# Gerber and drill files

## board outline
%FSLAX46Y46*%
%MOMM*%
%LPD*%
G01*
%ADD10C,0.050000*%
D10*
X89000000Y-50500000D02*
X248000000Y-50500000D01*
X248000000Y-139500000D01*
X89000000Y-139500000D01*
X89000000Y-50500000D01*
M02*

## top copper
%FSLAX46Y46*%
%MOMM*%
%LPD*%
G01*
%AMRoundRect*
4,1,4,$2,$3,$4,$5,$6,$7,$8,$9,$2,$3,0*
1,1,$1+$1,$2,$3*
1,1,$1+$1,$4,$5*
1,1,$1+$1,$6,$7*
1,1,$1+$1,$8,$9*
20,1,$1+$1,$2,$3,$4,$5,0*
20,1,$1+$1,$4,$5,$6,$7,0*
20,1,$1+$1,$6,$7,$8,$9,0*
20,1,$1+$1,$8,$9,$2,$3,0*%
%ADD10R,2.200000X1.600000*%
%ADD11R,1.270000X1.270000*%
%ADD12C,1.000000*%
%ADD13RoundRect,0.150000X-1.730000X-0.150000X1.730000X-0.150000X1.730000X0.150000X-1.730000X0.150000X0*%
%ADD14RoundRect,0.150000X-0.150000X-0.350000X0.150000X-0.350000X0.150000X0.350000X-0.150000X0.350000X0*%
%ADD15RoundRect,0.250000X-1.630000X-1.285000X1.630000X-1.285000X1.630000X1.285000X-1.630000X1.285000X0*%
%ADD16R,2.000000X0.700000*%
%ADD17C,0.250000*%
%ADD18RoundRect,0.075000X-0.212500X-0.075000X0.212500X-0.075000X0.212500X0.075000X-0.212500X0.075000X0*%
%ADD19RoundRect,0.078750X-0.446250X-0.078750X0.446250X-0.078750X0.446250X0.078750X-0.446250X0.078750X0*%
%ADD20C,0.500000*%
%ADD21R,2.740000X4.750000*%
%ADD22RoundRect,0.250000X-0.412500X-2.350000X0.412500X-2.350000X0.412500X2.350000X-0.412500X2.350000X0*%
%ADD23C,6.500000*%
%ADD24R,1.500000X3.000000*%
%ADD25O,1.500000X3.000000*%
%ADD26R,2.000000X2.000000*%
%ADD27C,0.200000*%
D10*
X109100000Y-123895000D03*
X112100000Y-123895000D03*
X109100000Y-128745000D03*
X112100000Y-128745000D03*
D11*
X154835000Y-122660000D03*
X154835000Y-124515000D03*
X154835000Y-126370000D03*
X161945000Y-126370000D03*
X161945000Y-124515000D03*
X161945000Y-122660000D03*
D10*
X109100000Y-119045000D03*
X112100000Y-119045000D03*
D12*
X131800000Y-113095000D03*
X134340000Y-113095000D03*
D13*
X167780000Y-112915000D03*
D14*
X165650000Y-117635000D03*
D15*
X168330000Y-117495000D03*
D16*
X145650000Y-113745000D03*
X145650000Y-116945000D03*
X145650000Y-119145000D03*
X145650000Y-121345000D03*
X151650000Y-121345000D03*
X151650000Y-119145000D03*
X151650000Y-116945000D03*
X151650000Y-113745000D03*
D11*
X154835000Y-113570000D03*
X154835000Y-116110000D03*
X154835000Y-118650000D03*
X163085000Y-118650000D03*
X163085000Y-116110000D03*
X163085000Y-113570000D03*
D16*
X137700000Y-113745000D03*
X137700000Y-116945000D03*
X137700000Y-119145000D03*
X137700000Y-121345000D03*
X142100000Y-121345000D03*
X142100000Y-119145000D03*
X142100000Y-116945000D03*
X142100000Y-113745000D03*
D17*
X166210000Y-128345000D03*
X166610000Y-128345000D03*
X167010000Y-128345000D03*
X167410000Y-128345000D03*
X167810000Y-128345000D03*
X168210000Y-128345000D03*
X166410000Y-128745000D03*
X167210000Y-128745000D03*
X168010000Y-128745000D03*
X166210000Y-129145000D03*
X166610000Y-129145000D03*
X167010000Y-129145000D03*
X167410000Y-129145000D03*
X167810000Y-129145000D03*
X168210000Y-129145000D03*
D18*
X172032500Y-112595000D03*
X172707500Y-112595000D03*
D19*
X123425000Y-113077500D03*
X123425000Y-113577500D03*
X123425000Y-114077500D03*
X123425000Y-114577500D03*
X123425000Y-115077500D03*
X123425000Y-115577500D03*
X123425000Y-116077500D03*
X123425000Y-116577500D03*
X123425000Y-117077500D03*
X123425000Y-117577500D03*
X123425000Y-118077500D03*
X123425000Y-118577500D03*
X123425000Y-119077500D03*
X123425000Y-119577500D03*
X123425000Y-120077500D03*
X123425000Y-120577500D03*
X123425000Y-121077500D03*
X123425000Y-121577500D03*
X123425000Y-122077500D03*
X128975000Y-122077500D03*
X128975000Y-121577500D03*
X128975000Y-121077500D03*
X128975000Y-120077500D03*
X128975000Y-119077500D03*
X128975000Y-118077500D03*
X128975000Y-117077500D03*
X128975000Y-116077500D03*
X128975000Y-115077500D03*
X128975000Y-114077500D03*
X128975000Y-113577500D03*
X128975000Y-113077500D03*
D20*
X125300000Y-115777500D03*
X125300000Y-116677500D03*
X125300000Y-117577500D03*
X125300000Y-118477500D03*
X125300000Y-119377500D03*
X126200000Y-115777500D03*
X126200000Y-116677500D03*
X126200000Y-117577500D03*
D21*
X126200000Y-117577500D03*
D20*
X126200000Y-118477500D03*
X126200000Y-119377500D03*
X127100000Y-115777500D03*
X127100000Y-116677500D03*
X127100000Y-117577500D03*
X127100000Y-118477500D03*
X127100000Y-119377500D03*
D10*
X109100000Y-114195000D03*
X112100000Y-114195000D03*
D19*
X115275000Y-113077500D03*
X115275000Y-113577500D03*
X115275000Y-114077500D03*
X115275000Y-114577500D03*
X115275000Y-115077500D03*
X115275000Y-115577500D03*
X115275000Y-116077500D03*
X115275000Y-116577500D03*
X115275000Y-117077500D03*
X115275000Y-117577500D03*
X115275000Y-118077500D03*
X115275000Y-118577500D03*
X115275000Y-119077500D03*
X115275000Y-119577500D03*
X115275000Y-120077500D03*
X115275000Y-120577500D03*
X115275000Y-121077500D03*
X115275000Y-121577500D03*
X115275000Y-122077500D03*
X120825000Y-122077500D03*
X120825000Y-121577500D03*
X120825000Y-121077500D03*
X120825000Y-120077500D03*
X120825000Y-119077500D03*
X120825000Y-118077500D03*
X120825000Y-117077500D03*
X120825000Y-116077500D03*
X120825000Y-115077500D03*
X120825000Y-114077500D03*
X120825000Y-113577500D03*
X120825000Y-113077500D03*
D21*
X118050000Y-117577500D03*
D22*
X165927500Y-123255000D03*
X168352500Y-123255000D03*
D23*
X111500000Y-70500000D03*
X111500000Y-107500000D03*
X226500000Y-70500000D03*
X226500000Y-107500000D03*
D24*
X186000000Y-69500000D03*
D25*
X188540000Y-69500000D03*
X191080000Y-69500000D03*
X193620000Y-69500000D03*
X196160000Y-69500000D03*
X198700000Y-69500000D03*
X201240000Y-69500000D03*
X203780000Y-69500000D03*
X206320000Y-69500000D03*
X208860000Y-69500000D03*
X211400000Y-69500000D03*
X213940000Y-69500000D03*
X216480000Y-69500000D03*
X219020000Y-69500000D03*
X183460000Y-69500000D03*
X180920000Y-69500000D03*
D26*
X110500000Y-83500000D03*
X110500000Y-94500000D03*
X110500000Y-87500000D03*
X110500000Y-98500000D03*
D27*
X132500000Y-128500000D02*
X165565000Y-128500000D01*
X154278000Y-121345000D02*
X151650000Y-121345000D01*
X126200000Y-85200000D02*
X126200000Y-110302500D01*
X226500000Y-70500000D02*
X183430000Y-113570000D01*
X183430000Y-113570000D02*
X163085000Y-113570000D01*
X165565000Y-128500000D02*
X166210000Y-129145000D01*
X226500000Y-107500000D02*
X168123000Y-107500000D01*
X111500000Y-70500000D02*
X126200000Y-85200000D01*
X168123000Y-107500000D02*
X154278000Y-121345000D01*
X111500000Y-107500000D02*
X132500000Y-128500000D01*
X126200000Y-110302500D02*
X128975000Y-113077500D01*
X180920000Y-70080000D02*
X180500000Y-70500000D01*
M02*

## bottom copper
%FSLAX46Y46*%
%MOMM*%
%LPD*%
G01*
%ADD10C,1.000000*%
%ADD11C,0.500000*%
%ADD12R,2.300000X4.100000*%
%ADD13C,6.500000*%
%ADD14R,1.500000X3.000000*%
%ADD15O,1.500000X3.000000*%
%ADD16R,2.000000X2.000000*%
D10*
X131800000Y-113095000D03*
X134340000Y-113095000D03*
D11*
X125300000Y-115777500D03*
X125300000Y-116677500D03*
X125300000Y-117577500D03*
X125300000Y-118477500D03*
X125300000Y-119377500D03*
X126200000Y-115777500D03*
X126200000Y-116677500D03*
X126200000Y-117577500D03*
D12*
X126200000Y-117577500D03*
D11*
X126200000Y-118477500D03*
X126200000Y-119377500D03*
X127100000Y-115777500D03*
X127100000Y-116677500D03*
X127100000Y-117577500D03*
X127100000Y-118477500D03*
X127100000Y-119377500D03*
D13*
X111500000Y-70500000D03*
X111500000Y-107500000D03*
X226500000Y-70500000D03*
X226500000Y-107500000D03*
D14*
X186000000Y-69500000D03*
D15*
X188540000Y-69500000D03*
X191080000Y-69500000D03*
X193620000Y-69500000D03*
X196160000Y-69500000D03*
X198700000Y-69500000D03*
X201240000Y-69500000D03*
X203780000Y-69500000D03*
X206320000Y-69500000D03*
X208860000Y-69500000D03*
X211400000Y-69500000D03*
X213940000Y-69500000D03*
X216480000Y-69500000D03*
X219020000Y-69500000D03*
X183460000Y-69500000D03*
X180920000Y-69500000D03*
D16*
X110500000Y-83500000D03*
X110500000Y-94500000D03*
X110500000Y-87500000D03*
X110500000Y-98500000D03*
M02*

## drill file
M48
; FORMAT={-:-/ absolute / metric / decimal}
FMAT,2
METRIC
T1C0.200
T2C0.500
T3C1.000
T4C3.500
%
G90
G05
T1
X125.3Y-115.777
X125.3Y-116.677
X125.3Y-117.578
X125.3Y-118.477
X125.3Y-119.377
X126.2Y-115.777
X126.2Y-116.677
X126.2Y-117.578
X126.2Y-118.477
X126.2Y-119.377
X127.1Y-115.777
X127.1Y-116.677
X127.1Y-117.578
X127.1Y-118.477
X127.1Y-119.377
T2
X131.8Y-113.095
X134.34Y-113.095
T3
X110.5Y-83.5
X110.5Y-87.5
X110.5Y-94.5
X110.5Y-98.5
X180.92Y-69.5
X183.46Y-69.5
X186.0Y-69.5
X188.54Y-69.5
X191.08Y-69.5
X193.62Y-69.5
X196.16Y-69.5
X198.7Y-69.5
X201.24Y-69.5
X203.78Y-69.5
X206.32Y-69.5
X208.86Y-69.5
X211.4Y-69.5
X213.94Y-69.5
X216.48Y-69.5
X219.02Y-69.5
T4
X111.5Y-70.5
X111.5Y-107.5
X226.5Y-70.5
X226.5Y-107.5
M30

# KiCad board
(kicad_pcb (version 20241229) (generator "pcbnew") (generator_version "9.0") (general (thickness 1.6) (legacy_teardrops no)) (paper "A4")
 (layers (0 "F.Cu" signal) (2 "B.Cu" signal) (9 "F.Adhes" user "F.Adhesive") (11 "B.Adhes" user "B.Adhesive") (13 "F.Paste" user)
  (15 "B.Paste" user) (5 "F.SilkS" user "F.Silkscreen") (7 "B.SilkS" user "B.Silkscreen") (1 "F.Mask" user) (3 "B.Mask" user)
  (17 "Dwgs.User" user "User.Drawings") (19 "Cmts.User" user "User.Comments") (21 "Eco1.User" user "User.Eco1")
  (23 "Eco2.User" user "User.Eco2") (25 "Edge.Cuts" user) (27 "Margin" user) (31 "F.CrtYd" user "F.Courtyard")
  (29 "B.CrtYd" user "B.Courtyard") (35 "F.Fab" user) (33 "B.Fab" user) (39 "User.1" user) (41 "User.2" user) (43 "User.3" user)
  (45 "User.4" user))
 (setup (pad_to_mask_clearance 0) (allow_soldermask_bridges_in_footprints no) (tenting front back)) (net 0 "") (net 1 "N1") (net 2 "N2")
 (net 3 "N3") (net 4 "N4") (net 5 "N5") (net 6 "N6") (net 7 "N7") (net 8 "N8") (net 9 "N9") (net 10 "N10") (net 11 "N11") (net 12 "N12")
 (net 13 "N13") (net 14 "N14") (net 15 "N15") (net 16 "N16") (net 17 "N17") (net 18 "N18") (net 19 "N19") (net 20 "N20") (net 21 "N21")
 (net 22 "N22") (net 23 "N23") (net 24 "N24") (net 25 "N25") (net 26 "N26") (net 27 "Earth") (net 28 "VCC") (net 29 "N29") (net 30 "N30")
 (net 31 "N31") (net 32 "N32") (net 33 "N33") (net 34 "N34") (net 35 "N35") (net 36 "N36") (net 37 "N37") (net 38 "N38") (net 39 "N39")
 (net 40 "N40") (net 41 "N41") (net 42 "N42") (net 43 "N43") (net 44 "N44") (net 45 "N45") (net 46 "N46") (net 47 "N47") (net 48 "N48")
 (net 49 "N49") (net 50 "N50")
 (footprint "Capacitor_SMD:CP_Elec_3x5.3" (layer "F.Cu") (at 110.6 123.895)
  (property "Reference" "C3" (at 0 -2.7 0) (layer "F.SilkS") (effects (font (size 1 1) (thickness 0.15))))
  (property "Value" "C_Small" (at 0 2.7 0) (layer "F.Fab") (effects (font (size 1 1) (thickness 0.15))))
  (pad "1" smd rect (at -1.5 0) (size 2.2 1.6) (layers "F.Cu" "F.Mask" "F.Paste") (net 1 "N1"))
  (pad "2" smd rect (at 1.5 0) (size 2.2 1.6) (layers "F.Cu" "F.Mask" "F.Paste") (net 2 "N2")))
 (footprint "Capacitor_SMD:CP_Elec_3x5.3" (layer "F.Cu") (at 110.6 128.745)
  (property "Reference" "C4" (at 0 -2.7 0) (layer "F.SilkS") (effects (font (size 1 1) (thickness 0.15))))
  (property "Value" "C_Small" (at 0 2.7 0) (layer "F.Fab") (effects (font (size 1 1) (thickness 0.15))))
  (pad "1" smd rect (at -1.5 0) (size 2.2 1.6) (layers "F.Cu" "F.Mask" "F.Paste") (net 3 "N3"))
  (pad "2" smd rect (at 1.5 0) (size 2.2 1.6) (layers "F.Cu" "F.Mask" "F.Paste") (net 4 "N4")))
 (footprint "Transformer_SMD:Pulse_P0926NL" (layer "F.Cu") (at 158.39 124.515)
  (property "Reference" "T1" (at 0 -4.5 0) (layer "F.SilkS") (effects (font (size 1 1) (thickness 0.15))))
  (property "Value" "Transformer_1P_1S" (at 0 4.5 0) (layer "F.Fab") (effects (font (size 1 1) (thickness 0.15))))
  (pad "1" smd rect (at -3.555 -1.855) (size 1.27 1.27) (layers "F.Cu" "F.Mask" "F.Paste") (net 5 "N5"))
  (pad "2" smd rect (at -3.555 0) (size 1.27 1.27) (layers "F.Cu" "F.Mask" "F.Paste") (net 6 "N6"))
  (pad "3" smd rect (at -3.555 1.855) (size 1.27 1.27) (layers "F.Cu" "F.Mask" "F.Paste") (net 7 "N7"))
  (pad "4" smd rect (at 3.555 1.855) (size 1.27 1.27) (layers "F.Cu" "F.Mask" "F.Paste") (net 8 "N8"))
  (pad "5" smd rect (at 3.555 0) (size 1.27 1.27) (layers "F.Cu" "F.Mask" "F.Paste"))
  (pad "6" smd rect (at 3.555 -1.855) (size 1.27 1.27) (layers "F.Cu" "F.Mask" "F.Paste")))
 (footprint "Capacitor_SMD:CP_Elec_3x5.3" (layer "F.Cu") (at 110.6 119.045)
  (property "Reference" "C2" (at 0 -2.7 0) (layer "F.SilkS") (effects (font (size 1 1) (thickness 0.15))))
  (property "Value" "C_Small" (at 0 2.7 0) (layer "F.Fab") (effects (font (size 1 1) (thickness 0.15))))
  (pad "1" smd rect (at -1.5 0) (size 2.2 1.6) (layers "F.Cu" "F.Mask" "F.Paste") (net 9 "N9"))
  (pad "2" smd rect (at 1.5 0) (size 2.2 1.6) (layers "F.Cu" "F.Mask" "F.Paste") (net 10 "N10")))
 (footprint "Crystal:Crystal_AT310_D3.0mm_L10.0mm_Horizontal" (layer "F.Cu") (at 131.8 113.095)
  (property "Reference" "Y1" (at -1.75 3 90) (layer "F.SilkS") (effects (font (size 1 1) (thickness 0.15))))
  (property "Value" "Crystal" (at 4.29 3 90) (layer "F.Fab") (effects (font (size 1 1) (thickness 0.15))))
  (pad "1" thru_hole circle (at 0 0) (size 1 1) (drill 0.5) (layers "*.Cu" "*.Mask") (remove_unused_layers no) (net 10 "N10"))
  (pad "2" thru_hole circle (at 2.54 0) (size 1 1) (drill 0.5) (layers "*.Cu" "*.Mask") (remove_unused_layers no) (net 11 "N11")))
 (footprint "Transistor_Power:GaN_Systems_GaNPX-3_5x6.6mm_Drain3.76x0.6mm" (layer "F.Cu") (at 167.78 115.825)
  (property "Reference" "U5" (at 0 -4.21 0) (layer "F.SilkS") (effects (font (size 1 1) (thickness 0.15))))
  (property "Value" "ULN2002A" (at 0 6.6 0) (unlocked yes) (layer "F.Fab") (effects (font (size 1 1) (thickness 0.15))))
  (pad "" smd roundrect (at -0.34 0.9525) (size 1.58 1.235) (layers "F.Paste") (roundrect_rratio 0.2024291498))
  (pad "" smd roundrect (at -0.34 2.3875) (size 1.58 1.235) (layers "F.Paste") (roundrect_rratio 0.2024291498))
  (pad "" smd roundrect (at 1.44 0.9525) (size 1.58 1.235) (layers "F.Paste") (roundrect_rratio 0.2024291498))
  (pad "" smd roundrect (at 1.44 2.3875) (size 1.58 1.235) (layers "F.Paste") (roundrect_rratio 0.2024291498))
  (pad "1" smd roundrect (at 0 -2.91) (size 3.76 0.6) (layers "F.Cu" "F.Mask" "F.Paste") (roundrect_rratio 0.25) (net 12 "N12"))
  (pad "2" smd roundrect (at -2.13 1.81) (size 0.6 1) (layers "F.Cu" "F.Mask" "F.Paste") (roundrect_rratio 0.25) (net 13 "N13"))
  (pad "3" smd roundrect (at 0.55 1.67) (size 3.76 3.07) (layers "F.Cu" "F.Mask") (roundrect_rratio 0.08143322476) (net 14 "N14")))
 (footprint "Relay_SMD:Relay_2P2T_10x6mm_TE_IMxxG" (layer "F.Cu") (at 148.65 117.545)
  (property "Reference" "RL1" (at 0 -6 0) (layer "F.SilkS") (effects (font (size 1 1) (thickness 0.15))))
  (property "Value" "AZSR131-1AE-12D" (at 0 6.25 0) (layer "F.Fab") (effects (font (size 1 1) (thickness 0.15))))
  (pad "1" smd rect (at -3 -3.8) (size 2 0.7) (layers "F.Cu" "F.Mask" "F.Paste") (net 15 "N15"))
  (pad "2" smd rect (at -3 -0.6) (size 2 0.7) (layers "F.Cu" "F.Mask" "F.Paste") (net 2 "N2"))
  (pad "3" smd rect (at -3 1.6) (size 2 0.7) (layers "F.Cu" "F.Mask" "F.Paste") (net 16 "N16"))
  (pad "4" smd rect (at -3 3.8) (size 2 0.7) (layers "F.Cu" "F.Mask" "F.Paste") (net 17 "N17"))
  (pad "5" smd rect (at 3 3.8) (size 2 0.7) (layers "F.Cu" "F.Mask" "F.Paste"))
  (pad "6" smd rect (at 3 1.6) (size 2 0.7) (layers "F.Cu" "F.Mask" "F.Paste"))
  (pad "7" smd rect (at 3 -0.6) (size 2 0.7) (layers "F.Cu" "F.Mask" "F.Paste"))
  (pad "8" smd rect (at 3 -3.8) (size 2 0.7) (layers "F.Cu" "F.Mask" "F.Paste")))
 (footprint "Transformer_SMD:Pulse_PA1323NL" (layer "F.Cu") (at 158.96 116.11)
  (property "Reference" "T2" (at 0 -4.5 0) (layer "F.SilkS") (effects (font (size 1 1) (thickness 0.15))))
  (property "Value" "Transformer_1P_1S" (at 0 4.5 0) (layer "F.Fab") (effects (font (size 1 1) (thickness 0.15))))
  (pad "1" smd rect (at -4.125 -2.54) (size 1.27 1.27) (layers "F.Cu" "F.Mask" "F.Paste") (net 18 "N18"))
  (pad "2" smd rect (at -4.125 0) (size 1.27 1.27) (layers "F.Cu" "F.Mask" "F.Paste") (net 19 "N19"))
  (pad "3" smd rect (at -4.125 2.54) (size 1.27 1.27) (layers "F.Cu" "F.Mask" "F.Paste") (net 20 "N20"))
  (pad "4" smd rect (at 4.125 2.54) (size 1.27 1.27) (layers "F.Cu" "F.Mask" "F.Paste") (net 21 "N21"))
  (pad "5" smd rect (at 4.125 0) (size 1.27 1.27) (layers "F.Cu" "F.Mask" "F.Paste"))
  (pad "6" smd rect (at 4.125 -2.54) (size 1.27 1.27) (layers "F.Cu" "F.Mask" "F.Paste")))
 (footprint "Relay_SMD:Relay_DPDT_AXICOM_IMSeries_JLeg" (layer "F.Cu") (at 139.9 117.545)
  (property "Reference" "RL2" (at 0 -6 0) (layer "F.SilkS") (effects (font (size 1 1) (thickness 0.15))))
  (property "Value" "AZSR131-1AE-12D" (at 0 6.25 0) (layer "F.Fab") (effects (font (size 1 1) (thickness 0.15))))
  (pad "1" smd rect (at -2.2 -3.8) (size 2 0.7) (layers "F.Cu" "F.Mask" "F.Paste") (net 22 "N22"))
  (pad "2" smd rect (at -2.2 -0.6) (size 2 0.7) (layers "F.Cu" "F.Mask" "F.Paste") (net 16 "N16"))
  (pad "3" smd rect (at -2.2 1.6) (size 2 0.7) (layers "F.Cu" "F.Mask" "F.Paste") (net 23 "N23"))
  (pad "4" smd rect (at -2.2 3.8) (size 2 0.7) (layers "F.Cu" "F.Mask" "F.Paste") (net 4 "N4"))
  (pad "5" smd rect (at 2.2 3.8) (size 2 0.7) (layers "F.Cu" "F.Mask" "F.Paste"))
  (pad "6" smd rect (at 2.2 1.6) (size 2 0.7) (layers "F.Cu" "F.Mask" "F.Paste"))
  (pad "7" smd rect (at 2.2 -0.6) (size 2 0.7) (layers "F.Cu" "F.Mask" "F.Paste"))
  (pad "8" smd rect (at 2.2 -3.8) (size 2 0.7) (layers "F.Cu" "F.Mask" "F.Paste")))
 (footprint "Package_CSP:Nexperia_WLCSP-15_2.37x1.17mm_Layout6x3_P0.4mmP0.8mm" (layer "F.Cu") (at 167.21 128.745)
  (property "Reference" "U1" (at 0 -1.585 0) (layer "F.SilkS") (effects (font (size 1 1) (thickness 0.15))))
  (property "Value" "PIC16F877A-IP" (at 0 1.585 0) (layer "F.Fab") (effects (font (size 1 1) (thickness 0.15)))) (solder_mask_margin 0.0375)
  (pad "A1" smd circle (at -1 -0.4) (size 0.25 0.25) (layers "F.Cu" "F.Mask" "F.Paste"))
  (pad "A2" smd circle (at -0.6 -0.4) (size 0.25 0.25) (layers "F.Cu" "F.Mask" "F.Paste"))
  (pad "A3" smd circle (at -0.2 -0.4) (size 0.25 0.25) (layers "F.Cu" "F.Mask" "F.Paste"))
  (pad "A4" smd circle (at 0.2 -0.4) (size 0.25 0.25) (layers "F.Cu" "F.Mask" "F.Paste"))
  (pad "A5" smd circle (at 0.6 -0.4) (size 0.25 0.25) (layers "F.Cu" "F.Mask" "F.Paste"))
  (pad "A6" smd circle (at 1 -0.4) (size 0.25 0.25) (layers "F.Cu" "F.Mask" "F.Paste"))
  (pad "B1" smd circle (at -0.8 0) (size 0.25 0.25) (layers "F.Cu" "F.Mask" "F.Paste"))
  (pad "B2" smd circle (at 0 0) (size 0.25 0.25) (layers "F.Cu" "F.Mask" "F.Paste"))
  (pad "B3" smd circle (at 0.8 0) (size 0.25 0.25) (layers "F.Cu" "F.Mask" "F.Paste"))
  (pad "C1" smd circle (at -1 0.4) (size 0.25 0.25) (layers "F.Cu" "F.Mask" "F.Paste"))
  (pad "C2" smd circle (at -0.6 0.4) (size 0.25 0.25) (layers "F.Cu" "F.Mask" "F.Paste"))
  (pad "C3" smd circle (at -0.2 0.4) (size 0.25 0.25) (layers "F.Cu" "F.Mask" "F.Paste"))
  (pad "C4" smd circle (at 0.2 0.4) (size 0.25 0.25) (layers "F.Cu" "F.Mask" "F.Paste"))
  (pad "C5" smd circle (at 0.6 0.4) (size 0.25 0.25) (layers "F.Cu" "F.Mask" "F.Paste"))
  (pad "C6" smd circle (at 1 0.4) (size 0.25 0.25) (layers "F.Cu" "F.Mask" "F.Paste")))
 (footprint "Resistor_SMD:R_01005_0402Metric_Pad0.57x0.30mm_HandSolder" (layer "F.Cu") (at 172.37 112.595)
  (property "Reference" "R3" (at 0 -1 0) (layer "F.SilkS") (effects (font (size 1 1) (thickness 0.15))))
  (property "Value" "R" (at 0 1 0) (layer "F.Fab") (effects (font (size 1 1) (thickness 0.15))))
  (pad "" smd roundrect (at -0.3625 0) (size 0.41 0.27) (layers "F.Paste") (roundrect_rratio 0.25))
  (pad "" smd roundrect (at 0.3625 0) (size 0.41 0.27) (layers "F.Paste") (roundrect_rratio 0.25))
  (pad "1" smd roundrect (at -0.3375 0) (size 0.575 0.3) (layers "F.Cu" "F.Mask") (roundrect_rratio 0.25) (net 19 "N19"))
  (pad "2" smd roundrect (at 0.3375 0) (size 0.575 0.3) (layers "F.Cu" "F.Mask") (roundrect_rratio 0.25) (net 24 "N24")))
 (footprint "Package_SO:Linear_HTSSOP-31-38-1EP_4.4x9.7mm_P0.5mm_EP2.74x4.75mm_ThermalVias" (layer "F.Cu") (at 126.2 117.5775)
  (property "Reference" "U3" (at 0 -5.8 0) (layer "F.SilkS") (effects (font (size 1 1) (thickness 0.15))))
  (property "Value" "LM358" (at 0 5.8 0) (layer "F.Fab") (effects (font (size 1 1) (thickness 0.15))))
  (pad "" smd roundrect (at -0.685 -1.58) (size 1.1 1.28) (layers "F.Paste") (roundrect_rratio 0.227273))
  (pad "" smd roundrect (at -0.685 0) (size 1.1 1.28) (layers "F.Paste") (roundrect_rratio 0.227273))
  (pad "" smd roundrect (at -0.685 1.58) (size 1.1 1.28) (layers "F.Paste") (roundrect_rratio 0.227273))
  (pad "" smd roundrect (at 0.685 -1.58) (size 1.1 1.28) (layers "F.Paste") (roundrect_rratio 0.227273))
  (pad "" smd roundrect (at 0.685 0) (size 1.1 1.28) (layers "F.Paste") (roundrect_rratio 0.227273))
  (pad "" smd roundrect (at 0.685 1.58) (size 1.1 1.28) (layers "F.Paste") (roundrect_rratio 0.227273))
  (pad "1" smd roundrect (at -2.775 -4.5) (size 1.05 0.315) (layers "F.Cu" "F.Mask" "F.Paste") (roundrect_rratio 0.25) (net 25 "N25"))
  (pad "2" smd roundrect (at -2.775 -4) (size 1.05 0.315) (layers "F.Cu" "F.Mask" "F.Paste") (roundrect_rratio 0.25) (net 5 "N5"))
  (pad "3" smd roundrect (at -2.775 -3.5) (size 1.05 0.315) (layers "F.Cu" "F.Mask" "F.Paste") (roundrect_rratio 0.25) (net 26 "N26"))
  (pad "4" smd roundrect (at -2.775 -3) (size 1.05 0.315) (layers "F.Cu" "F.Mask" "F.Paste") (roundrect_rratio 0.25) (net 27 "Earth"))
  (pad "5" smd roundrect (at -2.775 -2.5) (size 1.05 0.315) (layers "F.Cu" "F.Mask" "F.Paste") (roundrect_rratio 0.25))
  (pad "6" smd roundrect (at -2.775 -2) (size 1.05 0.315) (layers "F.Cu" "F.Mask" "F.Paste") (roundrect_rratio 0.25))
  (pad "7" smd roundrect (at -2.775 -1.5) (size 1.05 0.315) (layers "F.Cu" "F.Mask" "F.Paste") (roundrect_rratio 0.25))
  (pad "8" smd roundrect (at -2.775 -1) (size 1.05 0.315) (layers "F.Cu" "F.Mask" "F.Paste") (roundrect_rratio 0.25) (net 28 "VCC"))
  (pad "9" smd roundrect (at -2.775 -0.5) (size 1.05 0.315) (layers "F.Cu" "F.Mask" "F.Paste") (roundrect_rratio 0.25))
  (pad "10" smd roundrect (at -2.775 0) (size 1.05 0.315) (layers "F.Cu" "F.Mask" "F.Paste") (roundrect_rratio 0.25))
  (pad "11" smd roundrect (at -2.775 0.5) (size 1.05 0.315) (layers "F.Cu" "F.Mask" "F.Paste") (roundrect_rratio 0.25))
  (pad "12" smd roundrect (at -2.775 1) (size 1.05 0.315) (layers "F.Cu" "F.Mask" "F.Paste") (roundrect_rratio 0.25))
  (pad "13" smd roundrect (at -2.775 1.5) (size 1.05 0.315) (layers "F.Cu" "F.Mask" "F.Paste") (roundrect_rratio 0.25))
  (pad "14" smd roundrect (at -2.775 2) (size 1.05 0.315) (layers "F.Cu" "F.Mask" "F.Paste") (roundrect_rratio 0.25))
  (pad "15" smd roundrect (at -2.775 2.5) (size 1.05 0.315) (layers "F.Cu" "F.Mask" "F.Paste") (roundrect_rratio 0.25))
  (pad "16" smd roundrect (at -2.775 3) (size 1.05 0.315) (layers "F.Cu" "F.Mask" "F.Paste") (roundrect_rratio 0.25))
  (pad "17" smd roundrect (at -2.775 3.5) (size 1.05 0.315) (layers "F.Cu" "F.Mask" "F.Paste") (roundrect_rratio 0.25))
  (pad "18" smd roundrect (at -2.775 4) (size 1.05 0.315) (layers "F.Cu" "F.Mask" "F.Paste") (roundrect_rratio 0.25))
  (pad "19" smd roundrect (at -2.775 4.5) (size 1.05 0.315) (layers "F.Cu" "F.Mask" "F.Paste") (roundrect_rratio 0.25))
  (pad "20" smd roundrect (at 2.775 4.5) (size 1.05 0.315) (layers "F.Cu" "F.Mask" "F.Paste") (roundrect_rratio 0.25))
  (pad "21" smd roundrect (at 2.775 4) (size 1.05 0.315) (layers "F.Cu" "F.Mask" "F.Paste") (roundrect_rratio 0.25))
  (pad "22" smd roundrect (at 2.775 3.5) (size 1.05 0.315) (layers "F.Cu" "F.Mask" "F.Paste") (roundrect_rratio 0.25))
  (pad "24" smd roundrect (at 2.775 2.5) (size 1.05 0.315) (layers "F.Cu" "F.Mask" "F.Paste") (roundrect_rratio 0.25))
  (pad "26" smd roundrect (at 2.775 1.5) (size 1.05 0.315) (layers "F.Cu" "F.Mask" "F.Paste") (roundrect_rratio 0.25))
  (pad "28" smd roundrect (at 2.775 0.5) (size 1.05 0.315) (layers "F.Cu" "F.Mask" "F.Paste") (roundrect_rratio 0.25))
  (pad "30" smd roundrect (at 2.775 -0.5) (size 1.05 0.315) (layers "F.Cu" "F.Mask" "F.Paste") (roundrect_rratio 0.25))
  (pad "32" smd roundrect (at 2.775 -1.5) (size 1.05 0.315) (layers "F.Cu" "F.Mask" "F.Paste") (roundrect_rratio 0.25))
  (pad "34" smd roundrect (at 2.775 -2.5) (size 1.05 0.315) (layers "F.Cu" "F.Mask" "F.Paste") (roundrect_rratio 0.25))
  (pad "36" smd roundrect (at 2.775 -3.5) (size 1.05 0.315) (layers "F.Cu" "F.Mask" "F.Paste") (roundrect_rratio 0.25))
  (pad "37" smd roundrect (at 2.775 -4) (size 1.05 0.315) (layers "F.Cu" "F.Mask" "F.Paste") (roundrect_rratio 0.25))
  (pad "38" smd roundrect (at 2.775 -4.5) (size 1.05 0.315) (layers "F.Cu" "F.Mask" "F.Paste") (roundrect_rratio 0.25))
  (pad "39" thru_hole circle (at -0.9 -1.8) (size 0.5 0.5) (drill 0.2) (layers "*.Cu") (remove_unused_layers no))
  (pad "39" thru_hole circle (at -0.9 -0.9) (size 0.5 0.5) (drill 0.2) (layers "*.Cu") (remove_unused_layers no))
  (pad "39" thru_hole circle (at -0.9 0) (size 0.5 0.5) (drill 0.2) (layers "*.Cu") (remove_unused_layers no))
  (pad "39" thru_hole circle (at -0.9 0.9) (size 0.5 0.5) (drill 0.2) (layers "*.Cu") (remove_unused_layers no))
  (pad "39" thru_hole circle (at -0.9 1.8) (size 0.5 0.5) (drill 0.2) (layers "*.Cu") (remove_unused_layers no))
  (pad "39" thru_hole circle (at 0 -1.8) (size 0.5 0.5) (drill 0.2) (layers "*.Cu") (remove_unused_layers no))
  (pad "39" thru_hole circle (at 0 -0.9) (size 0.5 0.5) (drill 0.2) (layers "*.Cu") (remove_unused_layers no))
  (pad "39" thru_hole circle (at 0 0) (size 0.5 0.5) (drill 0.2) (layers "*.Cu") (remove_unused_layers no))
  (pad "39" smd rect (at 0 0) (size 2.3 4.1) (layers "B.Cu") (zone_connect 2))
  (pad "39" smd rect (at 0 0) (size 2.74 4.75) (layers "F.Cu" "F.Mask") (zone_connect 2))
  (pad "39" thru_hole circle (at 0 0.9) (size 0.5 0.5) (drill 0.2) (layers "*.Cu") (remove_unused_layers no))
  (pad "39" thru_hole circle (at 0 1.8) (size 0.5 0.5) (drill 0.2) (layers "*.Cu") (remove_unused_layers no))
  (pad "39" thru_hole circle (at 0.9 -1.8) (size 0.5 0.5) (drill 0.2) (layers "*.Cu") (remove_unused_layers no))
  (pad "39" thru_hole circle (at 0.9 -0.9) (size 0.5 0.5) (drill 0.2) (layers "*.Cu") (remove_unused_layers no))
  (pad "39" thru_hole circle (at 0.9 0) (size 0.5 0.5) (drill 0.2) (layers "*.Cu") (remove_unused_layers no))
  (pad "39" thru_hole circle (at 0.9 0.9) (size 0.5 0.5) (drill 0.2) (layers "*.Cu") (remove_unused_layers no))
  (pad "39" thru_hole circle (at 0.9 1.8) (size 0.5 0.5) (drill 0.2) (layers "*.Cu") (remove_unused_layers no)))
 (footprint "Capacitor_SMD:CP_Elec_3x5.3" (layer "F.Cu") (at 110.6 114.195)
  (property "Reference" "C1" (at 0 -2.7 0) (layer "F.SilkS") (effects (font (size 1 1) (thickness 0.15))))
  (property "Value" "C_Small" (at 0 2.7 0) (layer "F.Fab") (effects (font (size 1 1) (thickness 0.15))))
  (pad "1" smd rect (at -1.5 0) (size 2.2 1.6) (layers "F.Cu" "F.Mask" "F.Paste") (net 11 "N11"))
  (pad "2" smd rect (at 1.5 0) (size 2.2 1.6) (layers "F.Cu" "F.Mask" "F.Paste") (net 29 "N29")))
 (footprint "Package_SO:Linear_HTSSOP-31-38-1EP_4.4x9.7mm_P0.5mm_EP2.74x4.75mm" (layer "F.Cu") (at 118.05 117.5775)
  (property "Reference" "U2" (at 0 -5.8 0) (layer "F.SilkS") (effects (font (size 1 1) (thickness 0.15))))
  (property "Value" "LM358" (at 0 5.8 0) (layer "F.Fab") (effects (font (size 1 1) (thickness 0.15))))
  (pad "" smd roundrect (at -0.685 -1.58) (size 1.1 1.28) (layers "F.Paste") (roundrect_rratio 0.227273))
  (pad "" smd roundrect (at -0.685 0) (size 1.1 1.28) (layers "F.Paste") (roundrect_rratio 0.227273))
  (pad "" smd roundrect (at -0.685 1.58) (size 1.1 1.28) (layers "F.Paste") (roundrect_rratio 0.227273))
  (pad "" smd roundrect (at 0.685 -1.58) (size 1.1 1.28) (layers "F.Paste") (roundrect_rratio 0.227273))
  (pad "" smd roundrect (at 0.685 0) (size 1.1 1.28) (layers "F.Paste") (roundrect_rratio 0.227273))
  (pad "" smd roundrect (at 0.685 1.58) (size 1.1 1.28) (layers "F.Paste") (roundrect_rratio 0.227273))
  (pad "1" smd roundrect (at -2.775 -4.5) (size 1.05 0.315) (layers "F.Cu" "F.Mask" "F.Paste") (roundrect_rratio 0.25))
  (pad "2" smd roundrect (at -2.775 -4) (size 1.05 0.315) (layers "F.Cu" "F.Mask" "F.Paste") (roundrect_rratio 0.25))
  (pad "3" smd roundrect (at -2.775 -3.5) (size 1.05 0.315) (layers "F.Cu" "F.Mask" "F.Paste") (roundrect_rratio 0.25))
  (pad "4" smd roundrect (at -2.775 -3) (size 1.05 0.315) (layers "F.Cu" "F.Mask" "F.Paste") (roundrect_rratio 0.25) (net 27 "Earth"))
  (pad "5" smd roundrect (at -2.775 -2.5) (size 1.05 0.315) (layers "F.Cu" "F.Mask" "F.Paste") (roundrect_rratio 0.25) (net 24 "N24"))
  (pad "6" smd roundrect (at -2.775 -2) (size 1.05 0.315) (layers "F.Cu" "F.Mask" "F.Paste") (roundrect_rratio 0.25) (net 18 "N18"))
  (pad "7" smd roundrect (at -2.775 -1.5) (size 1.05 0.315) (layers "F.Cu" "F.Mask" "F.Paste") (roundrect_rratio 0.25) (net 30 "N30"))
  (pad "8" smd roundrect (at -2.775 -1) (size 1.05 0.315) (layers "F.Cu" "F.Mask" "F.Paste") (roundrect_rratio 0.25) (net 28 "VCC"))
  (pad "9" smd roundrect (at -2.775 -0.5) (size 1.05 0.315) (layers "F.Cu" "F.Mask" "F.Paste") (roundrect_rratio 0.25))
  (pad "10" smd roundrect (at -2.775 0) (size 1.05 0.315) (layers "F.Cu" "F.Mask" "F.Paste") (roundrect_rratio 0.25))
  (pad "11" smd roundrect (at -2.775 0.5) (size 1.05 0.315) (layers "F.Cu" "F.Mask" "F.Paste") (roundrect_rratio 0.25))
  (pad "12" smd roundrect (at -2.775 1) (size 1.05 0.315) (layers "F.Cu" "F.Mask" "F.Paste") (roundrect_rratio 0.25))
  (pad "13" smd roundrect (at -2.775 1.5) (size 1.05 0.315) (layers "F.Cu" "F.Mask" "F.Paste") (roundrect_rratio 0.25))
  (pad "14" smd roundrect (at -2.775 2) (size 1.05 0.315) (layers "F.Cu" "F.Mask" "F.Paste") (roundrect_rratio 0.25))
  (pad "15" smd roundrect (at -2.775 2.5) (size 1.05 0.315) (layers "F.Cu" "F.Mask" "F.Paste") (roundrect_rratio 0.25))
  (pad "16" smd roundrect (at -2.775 3) (size 1.05 0.315) (layers "F.Cu" "F.Mask" "F.Paste") (roundrect_rratio 0.25))
  (pad "17" smd roundrect (at -2.775 3.5) (size 1.05 0.315) (layers "F.Cu" "F.Mask" "F.Paste") (roundrect_rratio 0.25))
  (pad "18" smd roundrect (at -2.775 4) (size 1.05 0.315) (layers "F.Cu" "F.Mask" "F.Paste") (roundrect_rratio 0.25))
  (pad "19" smd roundrect (at -2.775 4.5) (size 1.05 0.315) (layers "F.Cu" "F.Mask" "F.Paste") (roundrect_rratio 0.25))
  (pad "20" smd roundrect (at 2.775 4.5) (size 1.05 0.315) (layers "F.Cu" "F.Mask" "F.Paste") (roundrect_rratio 0.25))
  (pad "21" smd roundrect (at 2.775 4) (size 1.05 0.315) (layers "F.Cu" "F.Mask" "F.Paste") (roundrect_rratio 0.25))
  (pad "22" smd roundrect (at 2.775 3.5) (size 1.05 0.315) (layers "F.Cu" "F.Mask" "F.Paste") (roundrect_rratio 0.25))
  (pad "24" smd roundrect (at 2.775 2.5) (size 1.05 0.315) (layers "F.Cu" "F.Mask" "F.Paste") (roundrect_rratio 0.25))
  (pad "26" smd roundrect (at 2.775 1.5) (size 1.05 0.315) (layers "F.Cu" "F.Mask" "F.Paste") (roundrect_rratio 0.25))
  (pad "28" smd roundrect (at 2.775 0.5) (size 1.05 0.315) (layers "F.Cu" "F.Mask" "F.Paste") (roundrect_rratio 0.25))
  (pad "30" smd roundrect (at 2.775 -0.5) (size 1.05 0.315) (layers "F.Cu" "F.Mask" "F.Paste") (roundrect_rratio 0.25))
  (pad "32" smd roundrect (at 2.775 -1.5) (size 1.05 0.315) (layers "F.Cu" "F.Mask" "F.Paste") (roundrect_rratio 0.25))
  (pad "34" smd roundrect (at 2.775 -2.5) (size 1.05 0.315) (layers "F.Cu" "F.Mask" "F.Paste") (roundrect_rratio 0.25))
  (pad "36" smd roundrect (at 2.775 -3.5) (size 1.05 0.315) (layers "F.Cu" "F.Mask" "F.Paste") (roundrect_rratio 0.25))
  (pad "37" smd roundrect (at 2.775 -4) (size 1.05 0.315) (layers "F.Cu" "F.Mask" "F.Paste") (roundrect_rratio 0.25))
  (pad "38" smd roundrect (at 2.775 -4.5) (size 1.05 0.315) (layers "F.Cu" "F.Mask" "F.Paste") (roundrect_rratio 0.25))
  (pad "39" smd rect (at 0 0) (size 2.74 4.75) (layers "F.Cu" "F.Mask") (zone_connect 2)))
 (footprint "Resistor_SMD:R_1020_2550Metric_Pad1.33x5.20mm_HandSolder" (layer "F.Cu") (at 167.14 123.255)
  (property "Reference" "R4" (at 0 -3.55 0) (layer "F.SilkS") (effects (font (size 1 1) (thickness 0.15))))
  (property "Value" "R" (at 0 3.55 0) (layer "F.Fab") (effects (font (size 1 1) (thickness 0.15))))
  (pad "1" smd roundrect (at -1.2125 0) (size 1.325 5.2) (layers "F.Cu" "F.Mask" "F.Paste") (roundrect_rratio 0.188679) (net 6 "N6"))
  (pad "2" smd roundrect (at 1.2125 0) (size 1.325 5.2) (layers "F.Cu" "F.Mask" "F.Paste") (roundrect_rratio 0.188679) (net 26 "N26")))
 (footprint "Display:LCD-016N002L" (layer "F.Cu") (at 186 69.5)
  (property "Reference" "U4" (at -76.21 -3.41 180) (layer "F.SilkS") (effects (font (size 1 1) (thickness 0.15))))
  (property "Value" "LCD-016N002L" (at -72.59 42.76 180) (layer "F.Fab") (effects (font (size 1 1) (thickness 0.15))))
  (pad "" thru_hole circle (at -74.5 1 180) (size 6.5 6.5) (drill 3.5) (layers "*.Cu" "*.Mask") (remove_unused_layers no))
  (pad "" thru_hole circle (at -74.5 38 180) (size 6.5 6.5) (drill 3.5) (layers "*.Cu" "*.Mask") (remove_unused_layers no))
  (pad "" thru_hole circle (at 40.5 1 180) (size 6.5 6.5) (drill 3.5) (layers "*.Cu" "*.Mask") (remove_unused_layers no))
  (pad "" thru_hole circle (at 40.5 38 180) (size 6.5 6.5) (drill 3.5) (layers "*.Cu" "*.Mask") (remove_unused_layers no))
  (pad "1" thru_hole rect (at 0 0 180) (size 1.5 3) (drill 1) (layers "*.Cu" "*.Mask") (remove_unused_layers no) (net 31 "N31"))
  (pad "2" thru_hole oval (at 2.54 0 180) (size 1.5 3) (drill 1) (layers "*.Cu" "*.Mask") (remove_unused_layers no) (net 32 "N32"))
  (pad "3" thru_hole oval (at 5.08 0 180) (size 1.5 3) (drill 1) (layers "*.Cu" "*.Mask") (remove_unused_layers no) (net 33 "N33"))
  (pad "4" thru_hole oval (at 7.62 0 180) (size 1.5 3) (drill 1) (layers "*.Cu" "*.Mask") (remove_unused_layers no) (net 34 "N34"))
  (pad "5" thru_hole oval (at 10.16 0 180) (size 1.5 3) (drill 1) (layers "*.Cu" "*.Mask") (remove_unused_layers no) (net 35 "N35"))
  (pad "6" thru_hole oval (at 12.7 0 180) (size 1.5 3) (drill 1) (layers "*.Cu" "*.Mask") (remove_unused_layers no) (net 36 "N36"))
  (pad "7" thru_hole oval (at 15.24 0 180) (size 1.5 3) (drill 1) (layers "*.Cu" "*.Mask") (remove_unused_layers no) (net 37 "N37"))
  (pad "8" thru_hole oval (at 17.78 0 180) (size 1.5 3) (drill 1) (layers "*.Cu" "*.Mask") (remove_unused_layers no) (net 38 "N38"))
  (pad "9" thru_hole oval (at 20.32 0 180) (size 1.5 3) (drill 1) (layers "*.Cu" "*.Mask") (remove_unused_layers no) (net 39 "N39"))
  (pad "10" thru_hole oval (at 22.86 0 180) (size 1.5 3) (drill 1) (layers "*.Cu" "*.Mask") (remove_unused_layers no) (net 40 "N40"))
  (pad "11" thru_hole oval (at 25.4 0 180) (size 1.5 3) (drill 1) (layers "*.Cu" "*.Mask") (remove_unused_layers no) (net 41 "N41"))
  (pad "12" thru_hole oval (at 27.94 0 180) (size 1.5 3) (drill 1) (layers "*.Cu" "*.Mask") (remove_unused_layers no) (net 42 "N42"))
  (pad "13" thru_hole oval (at 30.48 0 180) (size 1.5 3) (drill 1) (layers "*.Cu" "*.Mask") (remove_unused_layers no) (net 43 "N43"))
  (pad "14" thru_hole oval (at 33.02 0 180) (size 1.5 3) (drill 1) (layers "*.Cu" "*.Mask") (remove_unused_layers no) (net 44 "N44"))
  (pad "15" thru_hole oval (at -2.54 0 180) (size 1.5 3) (drill 1) (layers "*.Cu" "*.Mask") (remove_unused_layers no) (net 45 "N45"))
  (pad "16" thru_hole oval (at -5.08 0 180) (size 1.5 3) (drill 1) (layers "*.Cu" "*.Mask") (remove_unused_layers no) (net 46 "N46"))
  (pad "A1" thru_hole rect (at -75.5 14 180) (size 2 2) (drill 1) (layers "*.Cu" "*.Mask") (remove_unused_layers no) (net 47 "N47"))
  (pad "A2" thru_hole rect (at -75.5 25 180) (size 2 2) (drill 1) (layers "*.Cu" "*.Mask") (remove_unused_layers no) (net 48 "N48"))
  (pad "K1" thru_hole rect (at -75.5 18 180) (size 2 2) (drill 1) (layers "*.Cu" "*.Mask") (remove_unused_layers no) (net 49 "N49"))
  (pad "K2" thru_hole rect (at -75.5 29 180) (size 2 2) (drill 1) (layers "*.Cu" "*.Mask") (remove_unused_layers no) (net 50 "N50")))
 (gr_rect (start 89 50.5) (end 248 139.5) (stroke (width 0.05) (type default)) (fill no) (layer "Edge.Cuts"))
 (segment (start 132.5 128.5) (end 165.565 128.5) (width 0.2) (layer "F.Cu") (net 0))
 (segment (start 154.278 121.345) (end 151.65 121.345) (width 0.2) (layer "F.Cu") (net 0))
 (segment (start 126.2 85.2) (end 126.2 110.3025) (width 0.2) (layer "F.Cu") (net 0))
 (segment (start 226.5 70.5) (end 183.43 113.57) (width 0.2) (layer "F.Cu") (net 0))
 (segment (start 183.43 113.57) (end 163.085 113.57) (width 0.2) (layer "F.Cu") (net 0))
 (segment (start 165.565 128.5) (end 166.21 129.145) (width 0.2) (layer "F.Cu") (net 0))
 (segment (start 226.5 107.5) (end 168.123 107.5) (width 0.2) (layer "F.Cu") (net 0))
 (segment (start 111.5 70.5) (end 126.2 85.2) (width 0.2) (layer "F.Cu") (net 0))
 (segment (start 168.123 107.5) (end 154.278 121.345) (width 0.2) (layer "F.Cu") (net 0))
 (segment (start 111.5 107.5) (end 132.5 128.5) (width 0.2) (layer "F.Cu") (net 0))
 (segment (start 126.2 110.3025) (end 128.975 113.0775) (width 0.2) (layer "F.Cu") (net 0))
 (segment (start 180.92 70.08) (end 180.5 70.5) (width 0.2) (layer "F.Cu") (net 46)))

